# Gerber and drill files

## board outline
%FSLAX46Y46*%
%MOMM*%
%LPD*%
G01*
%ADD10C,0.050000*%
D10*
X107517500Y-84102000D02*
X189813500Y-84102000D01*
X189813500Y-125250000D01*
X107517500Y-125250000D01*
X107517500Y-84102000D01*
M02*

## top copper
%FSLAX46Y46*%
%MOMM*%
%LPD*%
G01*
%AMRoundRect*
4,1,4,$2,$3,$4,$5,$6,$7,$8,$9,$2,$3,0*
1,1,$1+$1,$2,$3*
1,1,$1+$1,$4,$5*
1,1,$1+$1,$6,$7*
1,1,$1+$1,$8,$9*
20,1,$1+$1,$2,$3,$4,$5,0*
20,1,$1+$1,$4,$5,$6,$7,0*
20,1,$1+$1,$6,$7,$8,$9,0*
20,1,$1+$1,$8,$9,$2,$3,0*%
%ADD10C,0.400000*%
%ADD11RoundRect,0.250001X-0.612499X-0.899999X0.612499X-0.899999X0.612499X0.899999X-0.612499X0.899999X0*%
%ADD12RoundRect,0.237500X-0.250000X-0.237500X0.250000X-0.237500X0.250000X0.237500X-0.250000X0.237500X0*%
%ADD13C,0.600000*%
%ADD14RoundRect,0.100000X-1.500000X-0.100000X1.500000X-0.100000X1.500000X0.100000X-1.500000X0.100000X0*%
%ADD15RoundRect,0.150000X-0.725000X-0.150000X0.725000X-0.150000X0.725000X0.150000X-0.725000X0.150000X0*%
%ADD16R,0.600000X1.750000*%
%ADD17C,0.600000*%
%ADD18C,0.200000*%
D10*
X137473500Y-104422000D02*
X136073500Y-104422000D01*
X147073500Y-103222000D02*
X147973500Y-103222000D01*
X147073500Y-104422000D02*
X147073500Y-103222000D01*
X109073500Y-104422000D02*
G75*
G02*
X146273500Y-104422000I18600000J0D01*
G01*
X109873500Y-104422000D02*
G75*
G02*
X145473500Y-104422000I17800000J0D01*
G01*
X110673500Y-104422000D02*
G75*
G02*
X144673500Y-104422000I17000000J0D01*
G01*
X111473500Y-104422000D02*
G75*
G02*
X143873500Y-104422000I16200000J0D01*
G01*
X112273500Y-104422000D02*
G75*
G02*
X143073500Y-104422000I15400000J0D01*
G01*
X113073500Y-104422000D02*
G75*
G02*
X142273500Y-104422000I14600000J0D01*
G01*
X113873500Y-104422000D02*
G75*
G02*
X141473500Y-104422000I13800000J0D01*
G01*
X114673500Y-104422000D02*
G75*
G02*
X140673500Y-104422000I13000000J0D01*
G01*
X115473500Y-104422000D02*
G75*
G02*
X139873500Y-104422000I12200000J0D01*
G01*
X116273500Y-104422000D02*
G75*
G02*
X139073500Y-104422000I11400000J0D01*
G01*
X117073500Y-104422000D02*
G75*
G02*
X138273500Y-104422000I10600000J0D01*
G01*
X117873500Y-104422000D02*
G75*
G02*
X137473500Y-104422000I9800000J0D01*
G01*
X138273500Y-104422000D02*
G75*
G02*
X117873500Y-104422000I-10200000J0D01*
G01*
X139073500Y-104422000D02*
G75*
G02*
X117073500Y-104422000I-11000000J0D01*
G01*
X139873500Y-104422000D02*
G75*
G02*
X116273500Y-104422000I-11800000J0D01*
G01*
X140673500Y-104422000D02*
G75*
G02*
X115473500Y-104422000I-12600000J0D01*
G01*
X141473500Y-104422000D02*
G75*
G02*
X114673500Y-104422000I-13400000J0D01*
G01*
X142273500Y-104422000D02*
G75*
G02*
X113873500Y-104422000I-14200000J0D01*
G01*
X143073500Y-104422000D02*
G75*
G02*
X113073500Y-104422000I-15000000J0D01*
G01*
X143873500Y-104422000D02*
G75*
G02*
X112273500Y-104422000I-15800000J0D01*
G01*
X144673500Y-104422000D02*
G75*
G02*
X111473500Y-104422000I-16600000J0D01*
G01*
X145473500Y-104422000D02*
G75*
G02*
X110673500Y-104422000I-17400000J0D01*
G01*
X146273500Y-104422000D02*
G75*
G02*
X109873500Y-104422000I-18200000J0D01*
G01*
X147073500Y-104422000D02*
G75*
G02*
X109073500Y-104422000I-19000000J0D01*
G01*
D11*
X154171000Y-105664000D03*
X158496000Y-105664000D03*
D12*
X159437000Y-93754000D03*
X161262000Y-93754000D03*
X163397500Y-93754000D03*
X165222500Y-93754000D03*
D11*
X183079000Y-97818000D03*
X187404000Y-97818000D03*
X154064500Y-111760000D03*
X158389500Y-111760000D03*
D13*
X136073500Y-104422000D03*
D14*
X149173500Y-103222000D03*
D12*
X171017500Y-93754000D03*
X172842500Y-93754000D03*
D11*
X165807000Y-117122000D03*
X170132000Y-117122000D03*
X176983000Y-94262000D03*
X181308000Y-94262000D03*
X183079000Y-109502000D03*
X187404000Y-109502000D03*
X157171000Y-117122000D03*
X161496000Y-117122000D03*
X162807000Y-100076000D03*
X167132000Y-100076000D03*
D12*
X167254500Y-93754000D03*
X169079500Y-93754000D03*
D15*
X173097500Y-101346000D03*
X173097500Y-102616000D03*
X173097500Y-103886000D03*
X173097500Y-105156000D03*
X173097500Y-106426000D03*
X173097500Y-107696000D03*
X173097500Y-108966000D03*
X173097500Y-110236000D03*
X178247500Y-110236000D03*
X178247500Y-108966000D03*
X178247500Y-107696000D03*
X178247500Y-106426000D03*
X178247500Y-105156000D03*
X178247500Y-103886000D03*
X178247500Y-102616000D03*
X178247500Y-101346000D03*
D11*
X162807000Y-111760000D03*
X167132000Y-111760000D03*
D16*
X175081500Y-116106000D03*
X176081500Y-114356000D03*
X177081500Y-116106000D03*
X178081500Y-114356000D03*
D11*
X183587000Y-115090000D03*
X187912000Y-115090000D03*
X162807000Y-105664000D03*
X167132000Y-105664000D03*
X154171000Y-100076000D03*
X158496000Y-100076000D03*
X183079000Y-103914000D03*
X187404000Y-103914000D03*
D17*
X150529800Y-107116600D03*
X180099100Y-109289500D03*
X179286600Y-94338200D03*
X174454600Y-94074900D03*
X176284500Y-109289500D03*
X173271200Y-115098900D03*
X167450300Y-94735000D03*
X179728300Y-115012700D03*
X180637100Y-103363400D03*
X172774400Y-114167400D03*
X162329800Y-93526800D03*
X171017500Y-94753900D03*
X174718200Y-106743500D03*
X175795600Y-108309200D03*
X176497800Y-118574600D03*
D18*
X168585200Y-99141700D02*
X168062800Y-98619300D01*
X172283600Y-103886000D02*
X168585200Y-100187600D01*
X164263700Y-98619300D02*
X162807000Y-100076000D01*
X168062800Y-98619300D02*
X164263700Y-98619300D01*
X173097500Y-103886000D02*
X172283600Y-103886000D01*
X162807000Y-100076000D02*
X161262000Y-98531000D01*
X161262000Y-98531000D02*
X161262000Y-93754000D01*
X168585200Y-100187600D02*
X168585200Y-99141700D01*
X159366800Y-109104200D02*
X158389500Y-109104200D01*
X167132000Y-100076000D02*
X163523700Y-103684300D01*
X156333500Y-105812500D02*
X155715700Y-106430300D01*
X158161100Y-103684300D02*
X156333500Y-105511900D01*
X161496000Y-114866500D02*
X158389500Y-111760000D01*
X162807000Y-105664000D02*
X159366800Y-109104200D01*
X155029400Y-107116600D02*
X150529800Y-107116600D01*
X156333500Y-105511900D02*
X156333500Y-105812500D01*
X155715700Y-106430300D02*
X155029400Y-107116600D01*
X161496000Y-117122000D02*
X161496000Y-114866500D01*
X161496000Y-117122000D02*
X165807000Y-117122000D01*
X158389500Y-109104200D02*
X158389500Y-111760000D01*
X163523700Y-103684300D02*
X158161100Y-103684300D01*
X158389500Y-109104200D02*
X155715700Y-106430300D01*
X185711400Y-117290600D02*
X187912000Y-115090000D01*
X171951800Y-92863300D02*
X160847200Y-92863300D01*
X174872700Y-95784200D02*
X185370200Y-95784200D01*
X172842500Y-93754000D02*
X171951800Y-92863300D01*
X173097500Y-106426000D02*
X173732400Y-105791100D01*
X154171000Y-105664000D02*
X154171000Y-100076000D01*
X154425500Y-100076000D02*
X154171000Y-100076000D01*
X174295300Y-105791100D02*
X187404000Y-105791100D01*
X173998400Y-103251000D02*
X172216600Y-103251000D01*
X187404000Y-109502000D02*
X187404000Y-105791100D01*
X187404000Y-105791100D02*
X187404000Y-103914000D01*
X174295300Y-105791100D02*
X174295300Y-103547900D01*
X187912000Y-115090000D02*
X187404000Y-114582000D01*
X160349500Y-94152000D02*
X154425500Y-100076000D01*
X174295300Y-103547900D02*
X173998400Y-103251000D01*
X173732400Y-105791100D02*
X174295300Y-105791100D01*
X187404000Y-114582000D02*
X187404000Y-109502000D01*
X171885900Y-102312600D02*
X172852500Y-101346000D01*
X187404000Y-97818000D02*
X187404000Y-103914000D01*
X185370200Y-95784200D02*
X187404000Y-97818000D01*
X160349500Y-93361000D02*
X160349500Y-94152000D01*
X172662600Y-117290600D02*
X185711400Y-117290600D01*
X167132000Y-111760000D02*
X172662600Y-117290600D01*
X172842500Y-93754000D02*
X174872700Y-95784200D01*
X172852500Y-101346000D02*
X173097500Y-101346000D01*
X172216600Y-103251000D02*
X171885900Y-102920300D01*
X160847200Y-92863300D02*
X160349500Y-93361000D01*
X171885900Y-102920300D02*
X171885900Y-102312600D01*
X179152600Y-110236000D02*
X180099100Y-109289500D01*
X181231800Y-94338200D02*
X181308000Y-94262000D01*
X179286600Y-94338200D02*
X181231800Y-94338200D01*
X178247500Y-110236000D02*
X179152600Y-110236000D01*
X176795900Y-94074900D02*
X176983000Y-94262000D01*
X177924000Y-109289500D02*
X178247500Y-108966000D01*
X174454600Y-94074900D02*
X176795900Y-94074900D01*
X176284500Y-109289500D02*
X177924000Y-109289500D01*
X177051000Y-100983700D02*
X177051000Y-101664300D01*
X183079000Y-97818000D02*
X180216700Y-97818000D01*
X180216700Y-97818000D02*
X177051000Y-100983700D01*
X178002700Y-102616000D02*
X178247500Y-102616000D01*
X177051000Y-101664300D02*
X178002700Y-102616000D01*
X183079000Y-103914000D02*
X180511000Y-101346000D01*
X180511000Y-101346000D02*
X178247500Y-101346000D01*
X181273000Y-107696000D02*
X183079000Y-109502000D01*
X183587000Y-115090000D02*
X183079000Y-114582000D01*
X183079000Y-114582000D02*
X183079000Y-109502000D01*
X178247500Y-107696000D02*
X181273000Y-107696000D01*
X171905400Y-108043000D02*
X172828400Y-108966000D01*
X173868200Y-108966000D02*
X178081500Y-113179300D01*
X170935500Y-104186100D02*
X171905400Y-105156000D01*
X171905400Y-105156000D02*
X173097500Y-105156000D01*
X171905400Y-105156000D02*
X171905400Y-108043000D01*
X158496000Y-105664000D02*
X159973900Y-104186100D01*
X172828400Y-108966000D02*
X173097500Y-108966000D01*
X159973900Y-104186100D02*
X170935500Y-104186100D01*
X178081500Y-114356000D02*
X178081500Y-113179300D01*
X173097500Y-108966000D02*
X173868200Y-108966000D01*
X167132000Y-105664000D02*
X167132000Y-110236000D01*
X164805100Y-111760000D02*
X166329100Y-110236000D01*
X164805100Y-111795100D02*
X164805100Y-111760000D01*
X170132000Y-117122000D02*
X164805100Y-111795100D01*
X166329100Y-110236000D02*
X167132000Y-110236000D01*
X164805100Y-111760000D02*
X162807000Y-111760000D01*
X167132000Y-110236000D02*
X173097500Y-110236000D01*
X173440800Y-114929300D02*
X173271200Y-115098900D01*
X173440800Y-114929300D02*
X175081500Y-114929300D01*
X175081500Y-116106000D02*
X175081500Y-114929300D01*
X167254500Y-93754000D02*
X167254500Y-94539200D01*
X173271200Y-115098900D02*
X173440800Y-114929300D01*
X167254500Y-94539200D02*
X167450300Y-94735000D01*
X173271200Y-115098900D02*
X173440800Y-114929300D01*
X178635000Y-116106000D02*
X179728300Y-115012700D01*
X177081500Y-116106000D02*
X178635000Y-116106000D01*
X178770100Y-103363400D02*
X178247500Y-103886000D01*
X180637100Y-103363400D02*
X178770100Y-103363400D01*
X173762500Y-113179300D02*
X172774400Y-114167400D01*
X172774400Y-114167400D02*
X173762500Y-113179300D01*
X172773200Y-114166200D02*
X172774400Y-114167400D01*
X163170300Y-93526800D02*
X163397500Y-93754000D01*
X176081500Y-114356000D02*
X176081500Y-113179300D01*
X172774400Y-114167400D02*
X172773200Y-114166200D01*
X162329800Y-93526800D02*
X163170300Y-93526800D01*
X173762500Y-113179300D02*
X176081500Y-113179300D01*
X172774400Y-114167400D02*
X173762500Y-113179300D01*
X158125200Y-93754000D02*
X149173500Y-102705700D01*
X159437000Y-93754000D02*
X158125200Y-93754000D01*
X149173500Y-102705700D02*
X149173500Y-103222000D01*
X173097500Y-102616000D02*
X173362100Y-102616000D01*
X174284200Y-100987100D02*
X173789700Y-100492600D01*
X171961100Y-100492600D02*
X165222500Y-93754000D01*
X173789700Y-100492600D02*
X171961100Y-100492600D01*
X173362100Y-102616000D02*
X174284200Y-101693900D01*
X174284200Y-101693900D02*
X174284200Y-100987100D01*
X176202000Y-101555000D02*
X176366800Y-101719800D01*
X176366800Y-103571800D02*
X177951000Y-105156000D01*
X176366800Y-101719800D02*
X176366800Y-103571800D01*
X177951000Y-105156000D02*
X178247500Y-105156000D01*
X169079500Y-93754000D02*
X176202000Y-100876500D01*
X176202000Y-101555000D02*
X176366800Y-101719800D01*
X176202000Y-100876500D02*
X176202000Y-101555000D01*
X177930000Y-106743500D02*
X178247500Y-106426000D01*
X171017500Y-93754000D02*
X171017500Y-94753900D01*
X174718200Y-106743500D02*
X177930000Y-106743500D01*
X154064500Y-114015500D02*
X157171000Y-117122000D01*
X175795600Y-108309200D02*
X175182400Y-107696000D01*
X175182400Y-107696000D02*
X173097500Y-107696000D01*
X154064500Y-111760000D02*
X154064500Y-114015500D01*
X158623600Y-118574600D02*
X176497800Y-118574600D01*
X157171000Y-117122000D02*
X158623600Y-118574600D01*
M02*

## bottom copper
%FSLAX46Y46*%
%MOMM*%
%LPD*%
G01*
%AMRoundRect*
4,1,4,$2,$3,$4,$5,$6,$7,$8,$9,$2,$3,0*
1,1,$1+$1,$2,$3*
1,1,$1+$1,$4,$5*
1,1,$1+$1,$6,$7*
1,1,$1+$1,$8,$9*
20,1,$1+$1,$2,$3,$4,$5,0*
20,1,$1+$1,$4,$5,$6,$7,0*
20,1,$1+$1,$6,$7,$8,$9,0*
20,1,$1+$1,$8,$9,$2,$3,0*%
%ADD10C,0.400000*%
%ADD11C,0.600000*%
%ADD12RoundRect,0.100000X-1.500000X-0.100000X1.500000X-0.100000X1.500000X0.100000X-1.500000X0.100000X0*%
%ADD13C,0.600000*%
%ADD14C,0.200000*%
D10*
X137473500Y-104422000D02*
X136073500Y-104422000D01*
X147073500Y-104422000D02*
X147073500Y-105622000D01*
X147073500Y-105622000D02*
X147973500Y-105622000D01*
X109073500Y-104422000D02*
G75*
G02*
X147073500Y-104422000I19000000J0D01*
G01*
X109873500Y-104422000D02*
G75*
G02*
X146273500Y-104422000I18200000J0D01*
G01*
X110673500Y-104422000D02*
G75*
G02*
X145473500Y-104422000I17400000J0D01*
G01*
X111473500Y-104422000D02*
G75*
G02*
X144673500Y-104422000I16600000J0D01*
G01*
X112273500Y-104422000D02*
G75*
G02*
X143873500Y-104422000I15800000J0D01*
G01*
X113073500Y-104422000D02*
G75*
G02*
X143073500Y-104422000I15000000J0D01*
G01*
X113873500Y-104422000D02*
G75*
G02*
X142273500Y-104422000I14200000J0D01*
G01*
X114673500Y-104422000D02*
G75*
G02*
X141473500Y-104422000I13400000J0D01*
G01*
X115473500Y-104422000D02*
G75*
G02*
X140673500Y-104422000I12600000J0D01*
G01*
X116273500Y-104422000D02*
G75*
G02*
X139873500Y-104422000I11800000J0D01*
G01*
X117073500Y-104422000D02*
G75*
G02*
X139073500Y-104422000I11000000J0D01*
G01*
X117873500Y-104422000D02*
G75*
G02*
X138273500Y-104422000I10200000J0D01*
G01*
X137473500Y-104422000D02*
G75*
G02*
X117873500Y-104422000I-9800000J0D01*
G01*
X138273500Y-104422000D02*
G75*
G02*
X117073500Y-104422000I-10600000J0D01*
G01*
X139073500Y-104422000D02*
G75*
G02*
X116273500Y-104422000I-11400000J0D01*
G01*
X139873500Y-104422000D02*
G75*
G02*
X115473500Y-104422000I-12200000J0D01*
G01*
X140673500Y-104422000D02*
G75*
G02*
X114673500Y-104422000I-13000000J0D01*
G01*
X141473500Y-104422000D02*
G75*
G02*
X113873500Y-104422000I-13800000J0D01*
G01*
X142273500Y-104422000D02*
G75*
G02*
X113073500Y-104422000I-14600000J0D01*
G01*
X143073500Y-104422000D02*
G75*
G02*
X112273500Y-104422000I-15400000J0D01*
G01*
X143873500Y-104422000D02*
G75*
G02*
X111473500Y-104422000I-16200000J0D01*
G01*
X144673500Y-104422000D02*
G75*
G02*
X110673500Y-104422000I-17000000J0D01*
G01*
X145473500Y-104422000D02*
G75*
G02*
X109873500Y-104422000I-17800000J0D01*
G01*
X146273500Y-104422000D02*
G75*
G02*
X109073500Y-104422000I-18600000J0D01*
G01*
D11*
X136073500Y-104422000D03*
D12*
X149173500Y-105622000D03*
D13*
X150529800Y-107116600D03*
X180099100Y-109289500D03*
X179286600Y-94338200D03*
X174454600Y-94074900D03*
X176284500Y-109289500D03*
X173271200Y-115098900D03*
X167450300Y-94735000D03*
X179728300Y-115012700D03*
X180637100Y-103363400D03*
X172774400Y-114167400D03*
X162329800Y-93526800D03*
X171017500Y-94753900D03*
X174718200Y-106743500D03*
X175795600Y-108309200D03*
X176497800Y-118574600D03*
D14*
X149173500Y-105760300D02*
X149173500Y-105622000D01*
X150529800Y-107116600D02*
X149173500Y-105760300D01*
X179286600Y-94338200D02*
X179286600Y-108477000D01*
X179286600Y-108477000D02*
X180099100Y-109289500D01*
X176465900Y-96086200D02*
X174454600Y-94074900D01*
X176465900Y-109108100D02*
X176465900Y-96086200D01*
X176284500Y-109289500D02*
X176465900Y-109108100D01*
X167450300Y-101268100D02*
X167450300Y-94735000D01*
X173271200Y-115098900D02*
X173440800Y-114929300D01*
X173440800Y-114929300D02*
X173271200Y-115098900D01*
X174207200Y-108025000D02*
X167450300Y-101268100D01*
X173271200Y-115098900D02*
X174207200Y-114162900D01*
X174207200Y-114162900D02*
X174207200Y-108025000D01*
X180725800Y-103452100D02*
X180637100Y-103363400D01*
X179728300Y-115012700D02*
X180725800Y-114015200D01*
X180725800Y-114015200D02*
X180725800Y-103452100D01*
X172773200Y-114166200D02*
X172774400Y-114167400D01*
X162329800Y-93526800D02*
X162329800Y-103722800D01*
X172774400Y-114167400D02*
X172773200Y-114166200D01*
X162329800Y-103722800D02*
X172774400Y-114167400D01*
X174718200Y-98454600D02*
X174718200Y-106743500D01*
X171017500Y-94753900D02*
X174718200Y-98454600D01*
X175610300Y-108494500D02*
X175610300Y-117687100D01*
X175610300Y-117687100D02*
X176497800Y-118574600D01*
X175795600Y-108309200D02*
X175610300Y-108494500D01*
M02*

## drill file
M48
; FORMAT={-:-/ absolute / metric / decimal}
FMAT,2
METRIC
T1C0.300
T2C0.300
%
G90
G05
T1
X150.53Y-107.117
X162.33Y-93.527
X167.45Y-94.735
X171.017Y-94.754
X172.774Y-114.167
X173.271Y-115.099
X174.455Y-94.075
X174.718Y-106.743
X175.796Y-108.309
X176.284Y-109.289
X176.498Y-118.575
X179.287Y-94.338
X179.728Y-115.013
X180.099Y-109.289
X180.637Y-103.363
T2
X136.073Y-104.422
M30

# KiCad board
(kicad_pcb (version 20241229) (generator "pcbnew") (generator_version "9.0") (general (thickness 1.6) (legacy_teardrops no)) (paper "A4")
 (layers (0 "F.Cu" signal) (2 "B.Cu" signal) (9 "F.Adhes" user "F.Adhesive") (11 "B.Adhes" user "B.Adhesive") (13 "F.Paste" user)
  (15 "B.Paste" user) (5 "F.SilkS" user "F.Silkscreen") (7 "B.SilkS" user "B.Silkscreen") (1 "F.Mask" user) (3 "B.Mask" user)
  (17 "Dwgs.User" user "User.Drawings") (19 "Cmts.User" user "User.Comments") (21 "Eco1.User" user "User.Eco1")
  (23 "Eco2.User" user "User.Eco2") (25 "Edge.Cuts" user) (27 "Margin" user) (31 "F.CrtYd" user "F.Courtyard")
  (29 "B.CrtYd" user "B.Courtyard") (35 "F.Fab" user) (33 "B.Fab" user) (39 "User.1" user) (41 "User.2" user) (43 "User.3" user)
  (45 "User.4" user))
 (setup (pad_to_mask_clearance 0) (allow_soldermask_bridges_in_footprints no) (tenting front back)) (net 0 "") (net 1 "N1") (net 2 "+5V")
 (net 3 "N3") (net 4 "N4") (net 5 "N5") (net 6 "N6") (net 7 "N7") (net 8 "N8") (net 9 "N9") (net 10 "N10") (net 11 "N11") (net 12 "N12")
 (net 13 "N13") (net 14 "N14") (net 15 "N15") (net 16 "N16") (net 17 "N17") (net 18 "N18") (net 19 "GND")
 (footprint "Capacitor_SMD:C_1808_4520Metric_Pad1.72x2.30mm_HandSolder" (layer "F.Cu") (at 156.3335 105.664)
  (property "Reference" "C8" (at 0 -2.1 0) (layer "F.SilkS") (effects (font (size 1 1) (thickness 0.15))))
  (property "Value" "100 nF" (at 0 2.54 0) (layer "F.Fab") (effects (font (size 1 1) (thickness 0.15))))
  (pad "1" smd roundrect (at -2.1625 0) (size 1.725 2.3) (layers "F.Cu" "F.Mask" "F.Paste") (roundrect_rratio 0.144928) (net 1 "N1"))
  (pad "2" smd roundrect (at 2.1625 0) (size 1.725 2.3) (layers "F.Cu" "F.Mask" "F.Paste") (roundrect_rratio 0.144928) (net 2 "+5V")))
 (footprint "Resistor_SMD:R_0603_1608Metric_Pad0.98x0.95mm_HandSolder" (layer "F.Cu") (at 160.3495 93.754)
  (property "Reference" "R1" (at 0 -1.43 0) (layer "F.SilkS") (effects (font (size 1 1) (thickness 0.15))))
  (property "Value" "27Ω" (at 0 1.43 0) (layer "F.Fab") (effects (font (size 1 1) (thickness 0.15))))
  (pad "1" smd roundrect (at -0.9125 0) (size 0.975 0.95) (layers "F.Cu" "F.Mask" "F.Paste") (roundrect_rratio 0.25) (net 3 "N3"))
  (pad "2" smd roundrect (at 0.9125 0) (size 0.975 0.95) (layers "F.Cu" "F.Mask" "F.Paste") (roundrect_rratio 0.25) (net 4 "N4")))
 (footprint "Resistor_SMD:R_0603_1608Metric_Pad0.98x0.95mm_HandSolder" (layer "F.Cu") (at 164.31 93.754)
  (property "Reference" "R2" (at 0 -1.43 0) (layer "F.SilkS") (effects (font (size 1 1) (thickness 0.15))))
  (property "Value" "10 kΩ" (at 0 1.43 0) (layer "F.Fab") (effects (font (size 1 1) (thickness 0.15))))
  (pad "1" smd roundrect (at -0.9125 0) (size 0.975 0.95) (layers "F.Cu" "F.Mask" "F.Paste") (roundrect_rratio 0.25) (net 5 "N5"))
  (pad "2" smd roundrect (at 0.9125 0) (size 0.975 0.95) (layers "F.Cu" "F.Mask" "F.Paste") (roundrect_rratio 0.25) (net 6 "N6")))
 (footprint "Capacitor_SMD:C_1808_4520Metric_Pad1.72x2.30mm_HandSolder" (layer "F.Cu") (at 185.2415 97.818)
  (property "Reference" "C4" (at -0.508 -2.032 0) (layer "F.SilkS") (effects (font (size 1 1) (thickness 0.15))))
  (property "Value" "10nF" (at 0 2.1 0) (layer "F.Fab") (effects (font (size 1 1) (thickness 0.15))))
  (pad "1" smd roundrect (at -2.1625 0) (size 1.725 2.3) (layers "F.Cu" "F.Mask" "F.Paste") (roundrect_rratio 0.144928) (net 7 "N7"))
  (pad "2" smd roundrect (at 2.1625 0) (size 1.725 2.3) (layers "F.Cu" "F.Mask" "F.Paste") (roundrect_rratio 0.144928) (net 1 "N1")))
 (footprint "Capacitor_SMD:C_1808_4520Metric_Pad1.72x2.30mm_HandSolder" (layer "F.Cu") (at 156.227 111.76)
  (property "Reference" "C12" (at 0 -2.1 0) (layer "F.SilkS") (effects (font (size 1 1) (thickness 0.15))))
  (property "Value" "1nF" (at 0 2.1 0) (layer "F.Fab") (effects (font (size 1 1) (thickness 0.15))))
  (pad "1" smd roundrect (at -2.1625 0) (size 1.725 2.3) (layers "F.Cu" "F.Mask" "F.Paste") (roundrect_rratio 0.144928) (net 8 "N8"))
  (pad "2" smd roundrect (at 2.1625 0) (size 1.725 2.3) (layers "F.Cu" "F.Mask" "F.Paste") (roundrect_rratio 0.144928) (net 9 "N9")))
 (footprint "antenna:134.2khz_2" (layer "F.Cu") (at 127.6735 104.422)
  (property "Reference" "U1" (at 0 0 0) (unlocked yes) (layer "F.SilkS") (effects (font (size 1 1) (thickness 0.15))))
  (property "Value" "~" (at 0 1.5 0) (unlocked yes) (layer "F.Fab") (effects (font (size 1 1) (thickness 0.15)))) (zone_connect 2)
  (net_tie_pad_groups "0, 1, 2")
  (fp_line (start 9.8 0) (end 8.4 0) (stroke (width 0.4) (type default)) (layer "F.Cu"))
  (fp_line (start 19.4 -1.2) (end 20.3 -1.2) (stroke (width 0.4) (type default)) (layer "F.Cu"))
  (fp_line (start 19.4 0) (end 19.4 -1.2) (stroke (width 0.4) (type default)) (layer "F.Cu"))
  (fp_arc (start -18.6 0) (mid 0 -18.6) (end 18.6 0) (stroke (width 0.4) (type default)) (layer "F.Cu"))
  (fp_arc (start -17.8 0) (mid 0 -17.8) (end 17.8 0) (stroke (width 0.4) (type default)) (layer "F.Cu"))
  (fp_arc (start -17 0) (mid 0 -17) (end 17 0) (stroke (width 0.4) (type default)) (layer "F.Cu"))
  (fp_arc (start -16.2 0) (mid 0 -16.2) (end 16.2 0) (stroke (width 0.4) (type default)) (layer "F.Cu"))
  (fp_arc (start -15.4 0) (mid 0 -15.4) (end 15.4 0) (stroke (width 0.4) (type default)) (layer "F.Cu"))
  (fp_arc (start -14.6 0) (mid 0 -14.6) (end 14.6 0) (stroke (width 0.4) (type default)) (layer "F.Cu"))
  (fp_arc (start -13.8 0) (mid 0 -13.8) (end 13.8 0) (stroke (width 0.4) (type default)) (layer "F.Cu"))
  (fp_arc (start -13 0) (mid 0 -13) (end 13 0) (stroke (width 0.4) (type default)) (layer "F.Cu"))
  (fp_arc (start -12.2 0) (mid 0 -12.2) (end 12.2 0) (stroke (width 0.4) (type default)) (layer "F.Cu"))
  (fp_arc (start -11.4 0) (mid 0 -11.4) (end 11.4 0) (stroke (width 0.4) (type default)) (layer "F.Cu"))
  (fp_arc (start -10.6 0) (mid 0 -10.6) (end 10.6 0) (stroke (width 0.4) (type default)) (layer "F.Cu"))
  (fp_arc (start -9.8 0) (mid 0 -9.8) (end 9.8 0) (stroke (width 0.4) (type default)) (layer "F.Cu"))
  (fp_arc (start 10.6 0) (mid 0.4 10.2) (end -9.8 0) (stroke (width 0.4) (type default)) (layer "F.Cu"))
  (fp_arc (start 11.4 0) (mid 0.4 11) (end -10.6 0) (stroke (width 0.4) (type default)) (layer "F.Cu"))
  (fp_arc (start 12.2 0) (mid 0.4 11.8) (end -11.4 0) (stroke (width 0.4) (type default)) (layer "F.Cu"))
  (fp_arc (start 13 0) (mid 0.4 12.6) (end -12.2 0) (stroke (width 0.4) (type default)) (layer "F.Cu"))
  (fp_arc (start 13.8 0) (mid 0.4 13.4) (end -13 0) (stroke (width 0.4) (type default)) (layer "F.Cu"))
  (fp_arc (start 14.6 0) (mid 0.4 14.2) (end -13.8 0) (stroke (width 0.4) (type default)) (layer "F.Cu"))
  (fp_arc (start 15.4 0) (mid 0.4 15) (end -14.6 0) (stroke (width 0.4) (type default)) (layer "F.Cu"))
  (fp_arc (start 16.2 0) (mid 0.4 15.8) (end -15.4 0) (stroke (width 0.4) (type default)) (layer "F.Cu"))
  (fp_arc (start 17 0) (mid 0.4 16.6) (end -16.2 0) (stroke (width 0.4) (type default)) (layer "F.Cu"))
  (fp_arc (start 17.8 0) (mid 0.4 17.4) (end -17 0) (stroke (width 0.4) (type default)) (layer "F.Cu"))
  (fp_arc (start 18.6 0) (mid 0.4 18.2) (end -17.8 0) (stroke (width 0.4) (type default)) (layer "F.Cu"))
  (fp_arc (start 19.4 0) (mid 0.4 19) (end -18.6 0) (stroke (width 0.4) (type default)) (layer "F.Cu"))
  (fp_line (start 9.8 0) (end 8.4 0) (stroke (width 0.4) (type default)) (layer "B.Cu"))
  (fp_line (start 19.4 0) (end 19.4 1.2) (stroke (width 0.4) (type default)) (layer "B.Cu"))
  (fp_line (start 19.4 1.2) (end 20.3 1.2) (stroke (width 0.4) (type default)) (layer "B.Cu"))
  (fp_arc (start -18.6 0) (mid 0.4 -19) (end 19.4 0) (stroke (width 0.4) (type default)) (layer "B.Cu"))
  (fp_arc (start -17.8 0) (mid 0.4 -18.2) (end 18.6 0) (stroke (width 0.4) (type default)) (layer "B.Cu"))
  (fp_arc (start -17 0) (mid 0.4 -17.4) (end 17.8 0) (stroke (width 0.4) (type default)) (layer "B.Cu"))
  (fp_arc (start -16.2 0) (mid 0.4 -16.6) (end 17 0) (stroke (width 0.4) (type default)) (layer "B.Cu"))
  (fp_arc (start -15.4 0) (mid 0.4 -15.8) (end 16.2 0) (stroke (width 0.4) (type default)) (layer "B.Cu"))
  (fp_arc (start -14.6 0) (mid 0.4 -15) (end 15.4 0) (stroke (width 0.4) (type default)) (layer "B.Cu"))
  (fp_arc (start -13.8 0) (mid 0.4 -14.2) (end 14.6 0) (stroke (width 0.4) (type default)) (layer "B.Cu"))
  (fp_arc (start -13 0) (mid 0.4 -13.4) (end 13.8 0) (stroke (width 0.4) (type default)) (layer "B.Cu"))
  (fp_arc (start -12.2 0) (mid 0.4 -12.6) (end 13 0) (stroke (width 0.4) (type default)) (layer "B.Cu"))
  (fp_arc (start -11.4 0) (mid 0.4 -11.8) (end 12.2 0) (stroke (width 0.4) (type default)) (layer "B.Cu"))
  (fp_arc (start -10.6 0) (mid 0.4 -11) (end 11.4 0) (stroke (width 0.4) (type default)) (layer "B.Cu"))
  (fp_arc (start -9.8 0) (mid 0.4 -10.2) (end 10.6 0) (stroke (width 0.4) (type default)) (layer "B.Cu"))
  (fp_arc (start 9.8 0) (mid 0 9.8) (end -9.8 0) (stroke (width 0.4) (type default)) (layer "B.Cu"))
  (fp_arc (start 10.6 0) (mid 0 10.6) (end -10.6 0) (stroke (width 0.4) (type default)) (layer "B.Cu"))
  (fp_arc (start 11.4 0) (mid 0 11.4) (end -11.4 0) (stroke (width 0.4) (type default)) (layer "B.Cu"))
  (fp_arc (start 12.2 0) (mid 0 12.2) (end -12.2 0) (stroke (width 0.4) (type default)) (layer "B.Cu"))
  (fp_arc (start 13 0) (mid 0 13) (end -13 0) (stroke (width 0.4) (type default)) (layer "B.Cu"))
  (fp_arc (start 13.8 0) (mid 0 13.8) (end -13.8 0) (stroke (width 0.4) (type default)) (layer "B.Cu"))
  (fp_arc (start 14.6 0) (mid 0 14.6) (end -14.6 0) (stroke (width 0.4) (type default)) (layer "B.Cu"))
  (fp_arc (start 15.4 0) (mid 0 15.4) (end -15.4 0) (stroke (width 0.4) (type default)) (layer "B.Cu"))
  (fp_arc (start 16.2 0) (mid 0 16.2) (end -16.2 0) (stroke (width 0.4) (type default)) (layer "B.Cu"))
  (fp_arc (start 17 0) (mid 0 17) (end -17 0) (stroke (width 0.4) (type default)) (layer "B.Cu"))
  (fp_arc (start 17.8 0) (mid 0 17.8) (end -17.8 0) (stroke (width 0.4) (type default)) (layer "B.Cu"))
  (fp_arc (start 18.6 0) (mid 0 18.6) (end -18.6 0) (stroke (width 0.4) (type default)) (layer "B.Cu"))
  (pad "0" thru_hole circle (at 8.4 0) (size 0.6 0.6) (drill 0.3) (layers "*.Cu") (remove_unused_layers yes) (keep_end_layers yes)
   (zone_layer_connections))
  (pad "1" smd roundrect (at 21.5 -1.2) (size 3.2 0.4) (layers "F.Cu") (roundrect_rratio 0.25) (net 3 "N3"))
  (pad "2" smd roundrect (at 21.5 1.2) (size 3.2 0.4) (layers "B.Cu") (roundrect_rratio 0.25) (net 9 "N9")))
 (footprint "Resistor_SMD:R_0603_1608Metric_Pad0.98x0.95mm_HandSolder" (layer "F.Cu") (at 171.93 93.754)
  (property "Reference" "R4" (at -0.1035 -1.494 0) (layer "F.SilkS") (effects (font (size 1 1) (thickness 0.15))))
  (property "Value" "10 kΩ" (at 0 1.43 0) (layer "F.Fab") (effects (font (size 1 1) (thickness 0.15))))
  (pad "1" smd roundrect (at -0.9125 0) (size 0.975 0.95) (layers "F.Cu" "F.Mask" "F.Paste") (roundrect_rratio 0.25) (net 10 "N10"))
  (pad "2" smd roundrect (at 0.9125 0) (size 0.975 0.95) (layers "F.Cu" "F.Mask" "F.Paste") (roundrect_rratio 0.25) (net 1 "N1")))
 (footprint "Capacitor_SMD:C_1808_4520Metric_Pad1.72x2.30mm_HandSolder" (layer "F.Cu") (at 167.9695 117.122)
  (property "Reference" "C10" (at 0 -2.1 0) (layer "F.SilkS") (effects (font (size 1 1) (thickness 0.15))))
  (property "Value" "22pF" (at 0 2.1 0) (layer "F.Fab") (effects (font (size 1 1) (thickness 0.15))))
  (pad "1" smd roundrect (at -2.1625 0) (size 1.725 2.3) (layers "F.Cu" "F.Mask" "F.Paste") (roundrect_rratio 0.144928) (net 9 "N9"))
  (pad "2" smd roundrect (at 2.1625 0) (size 1.725 2.3) (layers "F.Cu" "F.Mask" "F.Paste") (roundrect_rratio 0.144928) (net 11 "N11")))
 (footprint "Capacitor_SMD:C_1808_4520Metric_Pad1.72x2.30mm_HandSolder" (layer "F.Cu") (at 179.1455 94.262)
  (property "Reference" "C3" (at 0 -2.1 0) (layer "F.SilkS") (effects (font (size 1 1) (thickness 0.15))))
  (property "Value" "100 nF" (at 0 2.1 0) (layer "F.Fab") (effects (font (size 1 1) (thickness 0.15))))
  (pad "1" smd roundrect (at -2.1625 0) (size 1.725 2.3) (layers "F.Cu" "F.Mask" "F.Paste") (roundrect_rratio 0.144928) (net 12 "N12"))
  (pad "2" smd roundrect (at 2.1625 0) (size 1.725 2.3) (layers "F.Cu" "F.Mask" "F.Paste") (roundrect_rratio 0.144928) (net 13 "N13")))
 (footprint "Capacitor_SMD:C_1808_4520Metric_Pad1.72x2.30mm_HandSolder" (layer "F.Cu") (at 185.2415 109.502)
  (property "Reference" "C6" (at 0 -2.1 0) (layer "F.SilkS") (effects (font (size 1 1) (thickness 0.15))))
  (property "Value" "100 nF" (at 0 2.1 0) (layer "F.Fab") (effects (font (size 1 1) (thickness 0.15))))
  (pad "1" smd roundrect (at -2.1625 0) (size 1.725 2.3) (layers "F.Cu" "F.Mask" "F.Paste") (roundrect_rratio 0.144928) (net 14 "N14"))
  (pad "2" smd roundrect (at 2.1625 0) (size 1.725 2.3) (layers "F.Cu" "F.Mask" "F.Paste") (roundrect_rratio 0.144928) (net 1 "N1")))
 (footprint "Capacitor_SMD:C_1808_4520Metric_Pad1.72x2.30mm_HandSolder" (layer "F.Cu") (at 159.3335 117.122)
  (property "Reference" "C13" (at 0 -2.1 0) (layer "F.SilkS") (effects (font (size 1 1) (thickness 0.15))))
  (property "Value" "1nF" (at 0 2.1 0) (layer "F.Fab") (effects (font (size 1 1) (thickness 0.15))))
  (pad "1" smd roundrect (at -2.1625 0) (size 1.725 2.3) (layers "F.Cu" "F.Mask" "F.Paste") (roundrect_rratio 0.144928) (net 8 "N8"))
  (pad "2" smd roundrect (at 2.1625 0) (size 1.725 2.3) (layers "F.Cu" "F.Mask" "F.Paste") (roundrect_rratio 0.144928) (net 9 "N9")))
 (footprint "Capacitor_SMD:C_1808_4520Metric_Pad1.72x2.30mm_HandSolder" (layer "F.Cu") (at 164.9695 100.076)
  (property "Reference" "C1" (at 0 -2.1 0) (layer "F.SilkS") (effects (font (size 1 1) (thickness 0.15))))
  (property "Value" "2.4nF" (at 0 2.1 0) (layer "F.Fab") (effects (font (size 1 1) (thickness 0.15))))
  (pad "1" smd roundrect (at -2.1625 0) (size 1.725 2.3) (layers "F.Cu" "F.Mask" "F.Paste") (roundrect_rratio 0.144928) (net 4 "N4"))
  (pad "2" smd roundrect (at 2.1625 0) (size 1.725 2.3) (layers "F.Cu" "F.Mask" "F.Paste") (roundrect_rratio 0.144928) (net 9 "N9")))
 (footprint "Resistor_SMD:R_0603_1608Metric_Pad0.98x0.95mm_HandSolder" (layer "F.Cu") (at 168.167 93.754)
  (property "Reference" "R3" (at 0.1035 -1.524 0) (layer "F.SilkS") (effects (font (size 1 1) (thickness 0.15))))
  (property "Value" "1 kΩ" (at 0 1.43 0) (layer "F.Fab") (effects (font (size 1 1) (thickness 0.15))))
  (pad "1" smd roundrect (at -0.9125 0) (size 0.975 0.95) (layers "F.Cu" "F.Mask" "F.Paste") (roundrect_rratio 0.25) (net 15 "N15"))
  (pad "2" smd roundrect (at 0.9125 0) (size 0.975 0.95) (layers "F.Cu" "F.Mask" "F.Paste") (roundrect_rratio 0.25) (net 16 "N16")))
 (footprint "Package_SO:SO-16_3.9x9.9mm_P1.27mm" (layer "F.Cu") (at 175.6725 105.791)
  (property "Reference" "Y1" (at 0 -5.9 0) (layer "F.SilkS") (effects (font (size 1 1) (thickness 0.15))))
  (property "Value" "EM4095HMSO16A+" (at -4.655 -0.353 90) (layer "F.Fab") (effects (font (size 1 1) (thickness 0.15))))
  (pad "1" smd roundrect (at -2.575 -4.445) (size 1.75 0.6) (layers "F.Cu" "F.Mask" "F.Paste") (roundrect_rratio 0.25) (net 1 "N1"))
  (pad "2" smd roundrect (at -2.575 -3.175) (size 1.75 0.6) (layers "F.Cu" "F.Mask" "F.Paste") (roundrect_rratio 0.25) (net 6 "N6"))
  (pad "3" smd roundrect (at -2.575 -1.905) (size 1.75 0.6) (layers "F.Cu" "F.Mask" "F.Paste") (roundrect_rratio 0.25) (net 4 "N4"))
  (pad "4" smd roundrect (at -2.575 -0.635) (size 1.75 0.6) (layers "F.Cu" "F.Mask" "F.Paste") (roundrect_rratio 0.25) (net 2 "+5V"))
  (pad "5" smd roundrect (at -2.575 0.635) (size 1.75 0.6) (layers "F.Cu" "F.Mask" "F.Paste") (roundrect_rratio 0.25) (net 1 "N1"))
  (pad "6" smd roundrect (at -2.575 1.905) (size 1.75 0.6) (layers "F.Cu" "F.Mask" "F.Paste") (roundrect_rratio 0.25) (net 8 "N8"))
  (pad "7" smd roundrect (at -2.575 3.175) (size 1.75 0.6) (layers "F.Cu" "F.Mask" "F.Paste") (roundrect_rratio 0.25) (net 2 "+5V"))
  (pad "8" smd roundrect (at -2.575 4.445) (size 1.75 0.6) (layers "F.Cu" "F.Mask" "F.Paste") (roundrect_rratio 0.25) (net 11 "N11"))
  (pad "9" smd roundrect (at 2.575 4.445) (size 1.75 0.6) (layers "F.Cu" "F.Mask" "F.Paste") (roundrect_rratio 0.25) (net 13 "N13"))
  (pad "10" smd roundrect (at 2.575 3.175) (size 1.75 0.6) (layers "F.Cu" "F.Mask" "F.Paste") (roundrect_rratio 0.25) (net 12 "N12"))
  (pad "11" smd roundrect (at 2.575 1.905) (size 1.75 0.6) (layers "F.Cu" "F.Mask" "F.Paste") (roundrect_rratio 0.25) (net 14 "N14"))
  (pad "12" smd roundrect (at 2.575 0.635) (size 1.75 0.6) (layers "F.Cu" "F.Mask" "F.Paste") (roundrect_rratio 0.25) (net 10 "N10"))
  (pad "13" smd roundrect (at 2.575 -0.635) (size 1.75 0.6) (layers "F.Cu" "F.Mask" "F.Paste") (roundrect_rratio 0.25) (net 16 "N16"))
  (pad "14" smd roundrect (at 2.575 -1.905) (size 1.75 0.6) (layers "F.Cu" "F.Mask" "F.Paste") (roundrect_rratio 0.25) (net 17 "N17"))
  (pad "15" smd roundrect (at 2.575 -3.175) (size 1.75 0.6) (layers "F.Cu" "F.Mask" "F.Paste") (roundrect_rratio 0.25) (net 7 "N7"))
  (pad "16" smd roundrect (at 2.575 -4.445) (size 1.75 0.6) (layers "F.Cu" "F.Mask" "F.Paste") (roundrect_rratio 0.25) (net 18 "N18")))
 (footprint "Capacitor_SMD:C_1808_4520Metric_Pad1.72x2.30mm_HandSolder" (layer "F.Cu") (at 164.9695 111.76)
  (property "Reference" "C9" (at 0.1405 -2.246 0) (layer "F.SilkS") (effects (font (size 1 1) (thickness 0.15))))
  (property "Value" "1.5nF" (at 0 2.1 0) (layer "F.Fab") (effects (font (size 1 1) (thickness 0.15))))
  (pad "1" smd roundrect (at -2.1625 0) (size 1.725 2.3) (layers "F.Cu" "F.Mask" "F.Paste") (roundrect_rratio 0.144928) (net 11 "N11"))
  (pad "2" smd roundrect (at 2.1625 0) (size 1.725 2.3) (layers "F.Cu" "F.Mask" "F.Paste") (roundrect_rratio 0.144928) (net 1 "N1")))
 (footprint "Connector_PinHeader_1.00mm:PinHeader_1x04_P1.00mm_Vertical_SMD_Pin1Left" (layer "F.Cu") (at 176.5815 115.231 90)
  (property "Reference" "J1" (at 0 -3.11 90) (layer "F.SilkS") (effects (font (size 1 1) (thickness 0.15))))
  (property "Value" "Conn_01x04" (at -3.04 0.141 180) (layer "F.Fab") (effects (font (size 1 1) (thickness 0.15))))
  (pad "1" smd rect (at -0.875 -1.5 90) (size 1.75 0.6) (layers "F.Cu" "F.Mask" "F.Paste") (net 15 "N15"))
  (pad "2" smd rect (at 0.875 -0.5 90) (size 1.75 0.6) (layers "F.Cu" "F.Mask" "F.Paste") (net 5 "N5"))
  (pad "3" smd rect (at -0.875 0.5 90) (size 1.75 0.6) (layers "F.Cu" "F.Mask" "F.Paste") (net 17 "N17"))
  (pad "4" smd rect (at 0.875 1.5 90) (size 1.75 0.6) (layers "F.Cu" "F.Mask" "F.Paste") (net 2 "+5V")))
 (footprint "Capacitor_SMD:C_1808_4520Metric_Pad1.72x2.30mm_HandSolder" (layer "F.Cu") (at 185.7495 115.09)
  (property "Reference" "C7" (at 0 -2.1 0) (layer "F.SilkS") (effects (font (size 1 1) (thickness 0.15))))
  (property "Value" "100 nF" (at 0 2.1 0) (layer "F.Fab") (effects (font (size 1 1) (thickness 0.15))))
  (pad "1" smd roundrect (at -2.1625 0) (size 1.725 2.3) (layers "F.Cu" "F.Mask" "F.Paste") (roundrect_rratio 0.144928) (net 14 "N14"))
  (pad "2" smd roundrect (at 2.1625 0) (size 1.725 2.3) (layers "F.Cu" "F.Mask" "F.Paste") (roundrect_rratio 0.144928) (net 1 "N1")))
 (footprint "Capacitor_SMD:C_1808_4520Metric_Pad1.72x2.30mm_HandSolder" (layer "F.Cu") (at 164.9695 105.664)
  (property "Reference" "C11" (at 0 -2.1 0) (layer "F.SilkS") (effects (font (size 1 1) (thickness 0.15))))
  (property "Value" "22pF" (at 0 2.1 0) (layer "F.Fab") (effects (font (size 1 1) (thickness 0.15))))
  (pad "1" smd roundrect (at -2.1625 0) (size 1.725 2.3) (layers "F.Cu" "F.Mask" "F.Paste") (roundrect_rratio 0.144928) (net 9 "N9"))
  (pad "2" smd roundrect (at 2.1625 0) (size 1.725 2.3) (layers "F.Cu" "F.Mask" "F.Paste") (roundrect_rratio 0.144928) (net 11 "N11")))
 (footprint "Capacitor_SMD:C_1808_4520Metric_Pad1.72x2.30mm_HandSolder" (layer "F.Cu") (at 156.3335 100.076)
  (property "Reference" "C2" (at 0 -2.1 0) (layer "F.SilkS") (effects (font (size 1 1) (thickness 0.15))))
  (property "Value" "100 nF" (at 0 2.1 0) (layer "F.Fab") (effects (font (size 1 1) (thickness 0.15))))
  (pad "1" smd roundrect (at -2.1625 0) (size 1.725 2.3) (layers "F.Cu" "F.Mask" "F.Paste") (roundrect_rratio 0.144928) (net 1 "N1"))
  (pad "2" smd roundrect (at 2.1625 0) (size 1.725 2.3) (layers "F.Cu" "F.Mask" "F.Paste") (roundrect_rratio 0.144928) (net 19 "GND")))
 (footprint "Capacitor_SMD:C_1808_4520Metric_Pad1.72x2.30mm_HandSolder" (layer "F.Cu") (at 185.2415 103.914)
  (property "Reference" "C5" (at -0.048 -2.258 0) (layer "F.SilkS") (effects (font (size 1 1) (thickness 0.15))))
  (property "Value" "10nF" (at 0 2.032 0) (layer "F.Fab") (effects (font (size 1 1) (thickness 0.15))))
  (pad "1" smd roundrect (at -2.1625 0) (size 1.725 2.3) (layers "F.Cu" "F.Mask" "F.Paste") (roundrect_rratio 0.144928) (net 18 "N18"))
  (pad "2" smd roundrect (at 2.1625 0) (size 1.725 2.3) (layers "F.Cu" "F.Mask" "F.Paste") (roundrect_rratio 0.144928) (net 1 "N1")))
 (gr_rect (start 107.5175 84.102) (end 189.8135 125.25) (stroke (width 0.05) (type default)) (fill no) (layer "Edge.Cuts"))
 (segment (start 168.5852 99.1417) (end 168.0628 98.6193) (width 0.2) (layer "F.Cu") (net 4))
 (segment (start 172.2836 103.886) (end 168.5852 100.1876) (width 0.2) (layer "F.Cu") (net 4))
 (segment (start 164.2637 98.6193) (end 162.807 100.076) (width 0.2) (layer "F.Cu") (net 4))
 (segment (start 168.0628 98.6193) (end 164.2637 98.6193) (width 0.2) (layer "F.Cu") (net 4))
 (segment (start 173.0975 103.886) (end 172.2836 103.886) (width 0.2) (layer "F.Cu") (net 4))
 (segment (start 162.807 100.076) (end 161.262 98.531) (width 0.2) (layer "F.Cu") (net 4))
 (segment (start 161.262 98.531) (end 161.262 93.754) (width 0.2) (layer "F.Cu") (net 4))
 (segment (start 168.5852 100.1876) (end 168.5852 99.1417) (width 0.2) (layer "F.Cu") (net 4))
 (segment (start 159.3668 109.1042) (end 158.3895 109.1042) (width 0.2) (layer "F.Cu") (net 9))
 (segment (start 167.132 100.076) (end 163.5237 103.6843) (width 0.2) (layer "F.Cu") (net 9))
 (segment (start 156.3335 105.8125) (end 155.7157 106.4303) (width 0.2) (layer "F.Cu") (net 9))
 (segment (start 158.1611 103.6843) (end 156.3335 105.5119) (width 0.2) (layer "F.Cu") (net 9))
 (segment (start 161.496 114.8665) (end 158.3895 111.76) (width 0.2) (layer "F.Cu") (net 9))
 (segment (start 162.807 105.664) (end 159.3668 109.1042) (width 0.2) (layer "F.Cu") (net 9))
 (segment (start 155.0294 107.1166) (end 150.5298 107.1166) (width 0.2) (layer "F.Cu") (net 9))
 (segment (start 156.3335 105.5119) (end 156.3335 105.8125) (width 0.2) (layer "F.Cu") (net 9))
 (segment (start 155.7157 106.4303) (end 155.0294 107.1166) (width 0.2) (layer "F.Cu") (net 9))
 (segment (start 161.496 117.122) (end 161.496 114.8665) (width 0.2) (layer "F.Cu") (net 9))
 (segment (start 161.496 117.122) (end 165.807 117.122) (width 0.2) (layer "F.Cu") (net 9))
 (segment (start 158.3895 109.1042) (end 158.3895 111.76) (width 0.2) (layer "F.Cu") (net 9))
 (segment (start 163.5237 103.6843) (end 158.1611 103.6843) (width 0.2) (layer "F.Cu") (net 9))
 (segment (start 158.3895 109.1042) (end 155.7157 106.4303) (width 0.2) (layer "F.Cu") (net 9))
 (via (at 150.5298 107.1166) (size 0.6) (drill 0.3) (layers "F.Cu" "B.Cu") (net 9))
 (segment (start 149.1735 105.7603) (end 149.1735 105.622) (width 0.2) (layer "B.Cu") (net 9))
 (segment (start 150.5298 107.1166) (end 149.1735 105.7603) (width 0.2) (layer "B.Cu") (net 9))
 (segment (start 185.7114 117.2906) (end 187.912 115.09) (width 0.2) (layer "F.Cu") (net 1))
 (segment (start 171.9518 92.8633) (end 160.8472 92.8633) (width 0.2) (layer "F.Cu") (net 1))
 (segment (start 174.8727 95.7842) (end 185.3702 95.7842) (width 0.2) (layer "F.Cu") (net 1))
 (segment (start 172.8425 93.754) (end 171.9518 92.8633) (width 0.2) (layer "F.Cu") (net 1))
 (segment (start 173.0975 106.426) (end 173.7324 105.7911) (width 0.2) (layer "F.Cu") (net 1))
 (segment (start 154.171 105.664) (end 154.171 100.076) (width 0.2) (layer "F.Cu") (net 1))
 (segment (start 154.4255 100.076) (end 154.171 100.076) (width 0.2) (layer "F.Cu") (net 1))
 (segment (start 174.2953 105.7911) (end 187.404 105.7911) (width 0.2) (layer "F.Cu") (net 1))
 (segment (start 173.9984 103.251) (end 172.2166 103.251) (width 0.2) (layer "F.Cu") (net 1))
 (segment (start 187.404 109.502) (end 187.404 105.7911) (width 0.2) (layer "F.Cu") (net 1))
 (segment (start 187.404 105.7911) (end 187.404 103.914) (width 0.2) (layer "F.Cu") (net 1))
 (segment (start 174.2953 105.7911) (end 174.2953 103.5479) (width 0.2) (layer "F.Cu") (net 1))
 (segment (start 187.912 115.09) (end 187.404 114.582) (width 0.2) (layer "F.Cu") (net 1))
 (segment (start 160.3495 94.152) (end 154.4255 100.076) (width 0.2) (layer "F.Cu") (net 1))
 (segment (start 174.2953 103.5479) (end 173.9984 103.251) (width 0.2) (layer "F.Cu") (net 1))
 (segment (start 173.7324 105.7911) (end 174.2953 105.7911) (width 0.2) (layer "F.Cu") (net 1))
 (segment (start 187.404 114.582) (end 187.404 109.502) (width 0.2) (layer "F.Cu") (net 1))
 (segment (start 171.8859 102.3126) (end 172.8525 101.346) (width 0.2) (layer "F.Cu") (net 1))
 (segment (start 187.404 97.818) (end 187.404 103.914) (width 0.2) (layer "F.Cu") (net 1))
 (segment (start 185.3702 95.7842) (end 187.404 97.818) (width 0.2) (layer "F.Cu") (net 1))
 (segment (start 160.3495 93.361) (end 160.3495 94.152) (width 0.2) (layer "F.Cu") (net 1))
 (segment (start 172.6626 117.2906) (end 185.7114 117.2906) (width 0.2) (layer "F.Cu") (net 1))
 (segment (start 167.132 111.76) (end 172.6626 117.2906) (width 0.2) (layer "F.Cu") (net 1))
 (segment (start 172.8425 93.754) (end 174.8727 95.7842) (width 0.2) (layer "F.Cu") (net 1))
 (segment (start 172.8525 101.346) (end 173.0975 101.346) (width 0.2) (layer "F.Cu") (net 1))
 (segment (start 172.2166 103.251) (end 171.8859 102.9203) (width 0.2) (layer "F.Cu") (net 1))
 (segment (start 160.8472 92.8633) (end 160.3495 93.361) (width 0.2) (layer "F.Cu") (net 1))
 (segment (start 171.8859 102.9203) (end 171.8859 102.3126) (width 0.2) (layer "F.Cu") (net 1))
 (segment (start 179.1526 110.236) (end 180.0991 109.2895) (width 0.2) (layer "F.Cu") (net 13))
 (segment (start 181.2318 94.3382) (end 181.308 94.262) (width 0.2) (layer "F.Cu") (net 13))
 (segment (start 179.2866 94.3382) (end 181.2318 94.3382) (width 0.2) (layer "F.Cu") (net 13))
 (segment (start 178.2475 110.236) (end 179.1526 110.236) (width 0.2) (layer "F.Cu") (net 13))
 (via (at 180.0991 109.2895) (size 0.6) (drill 0.3) (layers "F.Cu" "B.Cu") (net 13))
 (via (at 179.2866 94.3382) (size 0.6) (drill 0.3) (layers "F.Cu" "B.Cu") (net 13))
 (segment (start 179.2866 94.3382) (end 179.2866 108.477) (width 0.2) (layer "B.Cu") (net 13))
 (segment (start 179.2866 108.477) (end 180.0991 109.2895) (width 0.2) (layer "B.Cu") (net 13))
 (segment (start 176.7959 94.0749) (end 176.983 94.262) (width 0.2) (layer "F.Cu") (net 12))
 (segment (start 177.924 109.2895) (end 178.2475 108.966) (width 0.2) (layer "F.Cu") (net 12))
 (segment (start 174.4546 94.0749) (end 176.7959 94.0749) (width 0.2) (layer "F.Cu") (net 12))
 (segment (start 176.2845 109.2895) (end 177.924 109.2895) (width 0.2) (layer "F.Cu") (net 12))
 (via (at 174.4546 94.0749) (size 0.6) (drill 0.3) (layers "F.Cu" "B.Cu") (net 12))
 (via (at 176.2845 109.2895) (size 0.6) (drill 0.3) (layers "F.Cu" "B.Cu") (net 12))
 (segment (start 176.4659 96.0862) (end 174.4546 94.0749) (width 0.2) (layer "B.Cu") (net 12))
 (segment (start 176.4659 109.1081) (end 176.4659 96.0862) (width 0.2) (layer "B.Cu") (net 12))
 (segment (start 176.2845 109.2895) (end 176.4659 109.1081) (width 0.2) (layer "B.Cu") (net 12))
 (segment (start 177.051 100.9837) (end 177.051 101.6643) (width 0.2) (layer "F.Cu") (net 7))
 (segment (start 183.079 97.818) (end 180.2167 97.818) (width 0.2) (layer "F.Cu") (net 7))
 (segment (start 180.2167 97.818) (end 177.051 100.9837) (width 0.2) (layer "F.Cu") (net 7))
 (segment (start 178.0027 102.616) (end 178.2475 102.616) (width 0.2) (layer "F.Cu") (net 7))
 (segment (start 177.051 101.6643) (end 178.0027 102.616) (width 0.2) (layer "F.Cu") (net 7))
 (segment (start 183.079 103.914) (end 180.511 101.346) (width 0.2) (layer "F.Cu") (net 18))
 (segment (start 180.511 101.346) (end 178.2475 101.346) (width 0.2) (layer "F.Cu") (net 18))
 (segment (start 181.273 107.696) (end 183.079 109.502) (width 0.2) (layer "F.Cu") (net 14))
 (segment (start 183.587 115.09) (end 183.079 114.582) (width 0.2) (layer "F.Cu") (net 14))
 (segment (start 183.079 114.582) (end 183.079 109.502) (width 0.2) (layer "F.Cu") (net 14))
 (segment (start 178.2475 107.696) (end 181.273 107.696) (width 0.2) (layer "F.Cu") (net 14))
 (segment (start 171.9054 108.043) (end 172.8284 108.966) (width 0.2) (layer "F.Cu") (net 2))
 (segment (start 173.8682 108.966) (end 178.0815 113.1793) (width 0.2) (layer "F.Cu") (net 2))
 (segment (start 170.9355 104.1861) (end 171.9054 105.156) (width 0.2) (layer "F.Cu") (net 2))
 (segment (start 171.9054 105.156) (end 173.0975 105.156) (width 0.2) (layer "F.Cu") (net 2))
 (segment (start 171.9054 105.156) (end 171.9054 108.043) (width 0.2) (layer "F.Cu") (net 2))
 (segment (start 158.496 105.664) (end 159.9739 104.1861) (width 0.2) (layer "F.Cu") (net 2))
 (segment (start 172.8284 108.966) (end 173.0975 108.966) (width 0.2) (layer "F.Cu") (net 2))
 (segment (start 159.9739 104.1861) (end 170.9355 104.1861) (width 0.2) (layer "F.Cu") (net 2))
 (segment (start 178.0815 114.356) (end 178.0815 113.1793) (width 0.2) (layer "F.Cu") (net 2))
 (segment (start 173.0975 108.966) (end 173.8682 108.966) (width 0.2) (layer "F.Cu") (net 2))
 (segment (start 167.132 105.664) (end 167.132 110.236) (width 0.2) (layer "F.Cu") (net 11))
 (segment (start 164.8051 111.76) (end 166.3291 110.236) (width 0.2) (layer "F.Cu") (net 11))
 (segment (start 164.8051 111.7951) (end 164.8051 111.76) (width 0.2) (layer "F.Cu") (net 11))
 (segment (start 170.132 117.122) (end 164.8051 111.7951) (width 0.2) (layer "F.Cu") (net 11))
 (segment (start 166.3291 110.236) (end 167.132 110.236) (width 0.2) (layer "F.Cu") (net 11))
 (segment (start 164.8051 111.76) (end 162.807 111.76) (width 0.2) (layer "F.Cu") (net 11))
 (segment (start 167.132 110.236) (end 173.0975 110.236) (width 0.2) (layer "F.Cu") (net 11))
 (segment (start 173.4408 114.9293) (end 173.2712 115.0989) (width 0.2) (layer "F.Cu") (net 15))
 (segment (start 173.4408 114.9293) (end 175.0815 114.9293) (width 0.2) (layer "F.Cu") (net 15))
 (segment (start 175.0815 116.106) (end 175.0815 114.9293) (width 0.2) (layer "F.Cu") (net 15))
 (segment (start 167.2545 93.754) (end 167.2545 94.5392) (width 0.2) (layer "F.Cu") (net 15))
 (segment (start 173.2712 115.0989) (end 173.4408 114.9293) (width 0.2) (layer "F.Cu") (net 15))
 (segment (start 167.2545 94.5392) (end 167.4503 94.735) (width 0.2) (layer "F.Cu") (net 15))
 (segment (start 173.2712 115.0989) (end 173.4408 114.9293) (width 0.2) (layer "F.Cu") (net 15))
 (via (at 173.2712 115.0989) (size 0.6) (drill 0.3) (layers "F.Cu" "B.Cu") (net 15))
 (via (at 167.4503 94.735) (size 0.6) (drill 0.3) (layers "F.Cu" "B.Cu") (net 15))
 (segment (start 167.4503 101.2681) (end 167.4503 94.735) (width 0.2) (layer "B.Cu") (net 15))
 (segment (start 173.2712 115.0989) (end 173.4408 114.9293) (width 0.2) (layer "B.Cu") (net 15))
 (segment (start 173.4408 114.9293) (end 173.2712 115.0989) (width 0.2) (layer "B.Cu") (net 15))
 (segment (start 174.2072 108.025) (end 167.4503 101.2681) (width 0.2) (layer "B.Cu") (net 15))
 (segment (start 173.2712 115.0989) (end 174.2072 114.1629) (width 0.2) (layer "B.Cu") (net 15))
 (segment (start 174.2072 114.1629) (end 174.2072 108.025) (width 0.2) (layer "B.Cu") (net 15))
 (segment (start 178.635 116.106) (end 179.7283 115.0127) (width 0.2) (layer "F.Cu") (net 17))
 (segment (start 177.0815 116.106) (end 178.635 116.106) (width 0.2) (layer "F.Cu") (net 17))
 (segment (start 178.7701 103.3634) (end 178.2475 103.886) (width 0.2) (layer "F.Cu") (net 17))
 (segment (start 180.6371 103.3634) (end 178.7701 103.3634) (width 0.2) (layer "F.Cu") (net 17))
 (via (at 179.7283 115.0127) (size 0.6) (drill 0.3) (layers "F.Cu" "B.Cu") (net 17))
 (via (at 180.6371 103.3634) (size 0.6) (drill 0.3) (layers "F.Cu" "B.Cu") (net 17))
 (segment (start 180.7258 103.4521) (end 180.6371 103.3634) (width 0.2) (layer "B.Cu") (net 17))
 (segment (start 179.7283 115.0127) (end 180.7258 114.0152) (width 0.2) (layer "B.Cu") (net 17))
 (segment (start 180.7258 114.0152) (end 180.7258 103.4521) (width 0.2) (layer "B.Cu") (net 17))
 (segment (start 173.7625 113.1793) (end 172.7744 114.1674) (width 0.2) (layer "F.Cu") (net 5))
 (segment (start 172.7744 114.1674) (end 173.7625 113.1793) (width 0.2) (layer "F.Cu") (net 5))
 (segment (start 172.7732 114.1662) (end 172.7744 114.1674) (width 0.2) (layer "F.Cu") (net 5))
 (segment (start 163.1703 93.5268) (end 163.3975 93.754) (width 0.2) (layer "F.Cu") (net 5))
 (segment (start 176.0815 114.356) (end 176.0815 113.1793) (width 0.2) (layer "F.Cu") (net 5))
 (segment (start 172.7744 114.1674) (end 172.7732 114.1662) (width 0.2) (layer "F.Cu") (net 5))
 (segment (start 162.3298 93.5268) (end 163.1703 93.5268) (width 0.2) (layer "F.Cu") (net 5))
 (segment (start 173.7625 113.1793) (end 176.0815 113.1793) (width 0.2) (layer "F.Cu") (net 5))
 (segment (start 172.7744 114.1674) (end 173.7625 113.1793) (width 0.2) (layer "F.Cu") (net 5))
 (via (at 172.7744 114.1674) (size 0.6) (drill 0.3) (layers "F.Cu" "B.Cu") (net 5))
 (via (at 162.3298 93.5268) (size 0.6) (drill 0.3) (layers "F.Cu" "B.Cu") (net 5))
 (segment (start 172.7732 114.1662) (end 172.7744 114.1674) (width 0.2) (layer "B.Cu") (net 5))
 (segment (start 162.3298 93.5268) (end 162.3298 103.7228) (width 0.2) (layer "B.Cu") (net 5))
 (segment (start 172.7744 114.1674) (end 172.7732 114.1662) (width 0.2) (layer "B.Cu") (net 5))
 (segment (start 162.3298 103.7228) (end 172.7744 114.1674) (width 0.2) (layer "B.Cu") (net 5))
 (segment (start 158.1252 93.754) (end 149.1735 102.7057) (width 0.2) (layer "F.Cu") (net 3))
 (segment (start 159.437 93.754) (end 158.1252 93.754) (width 0.2) (layer "F.Cu") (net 3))
 (segment (start 149.1735 102.7057) (end 149.1735 103.222) (width 0.2) (layer "F.Cu") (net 3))
 (segment (start 173.0975 102.616) (end 173.3621 102.616) (width 0.2) (layer "F.Cu") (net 6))
 (segment (start 174.2842 100.9871) (end 173.7897 100.4926) (width 0.2) (layer "F.Cu") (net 6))
 (segment (start 171.9611 100.4926) (end 165.2225 93.754) (width 0.2) (layer "F.Cu") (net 6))
 (segment (start 173.7897 100.4926) (end 171.9611 100.4926) (width 0.2) (layer "F.Cu") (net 6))
 (segment (start 173.3621 102.616) (end 174.2842 101.6939) (width 0.2) (layer "F.Cu") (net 6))
 (segment (start 174.2842 101.6939) (end 174.2842 100.9871) (width 0.2) (layer "F.Cu") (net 6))
 (segment (start 176.202 101.555) (end 176.3668 101.7198) (width 0.2) (layer "F.Cu") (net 16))
 (segment (start 176.3668 103.5718) (end 177.951 105.156) (width 0.2) (layer "F.Cu") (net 16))
 (segment (start 176.3668 101.7198) (end 176.3668 103.5718) (width 0.2) (layer "F.Cu") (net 16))
 (segment (start 177.951 105.156) (end 178.2475 105.156) (width 0.2) (layer "F.Cu") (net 16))
 (segment (start 169.0795 93.754) (end 176.202 100.8765) (width 0.2) (layer "F.Cu") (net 16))
 (segment (start 176.202 101.555) (end 176.3668 101.7198) (width 0.2) (layer "F.Cu") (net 16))
 (segment (start 176.202 100.8765) (end 176.202 101.555) (width 0.2) (layer "F.Cu") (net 16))
 (segment (start 177.93 106.7435) (end 178.2475 106.426) (width 0.2) (layer "F.Cu") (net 10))
 (segment (start 171.0175 93.754) (end 171.0175 94.7539) (width 0.2) (layer "F.Cu") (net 10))
 (segment (start 174.7182 106.7435) (end 177.93 106.7435) (width 0.2) (layer "F.Cu") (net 10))
 (via (at 171.0175 94.7539) (size 0.6) (drill 0.3) (layers "F.Cu" "B.Cu") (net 10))
 (via (at 174.7182 106.7435) (size 0.6) (drill 0.3) (layers "F.Cu" "B.Cu") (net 10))
 (segment (start 174.7182 98.4546) (end 174.7182 106.7435) (width 0.2) (layer "B.Cu") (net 10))
 (segment (start 171.0175 94.7539) (end 174.7182 98.4546) (width 0.2) (layer "B.Cu") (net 10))
 (segment (start 154.0645 114.0155) (end 157.171 117.122) (width 0.2) (layer "F.Cu") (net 8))
 (segment (start 175.7956 108.3092) (end 175.1824 107.696) (width 0.2) (layer "F.Cu") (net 8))
 (segment (start 175.1824 107.696) (end 173.0975 107.696) (width 0.2) (layer "F.Cu") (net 8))
 (segment (start 154.0645 111.76) (end 154.0645 114.0155) (width 0.2) (layer "F.Cu") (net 8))
 (segment (start 158.6236 118.5746) (end 176.4978 118.5746) (width 0.2) (layer "F.Cu") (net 8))
 (segment (start 157.171 117.122) (end 158.6236 118.5746) (width 0.2) (layer "F.Cu") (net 8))
 (via (at 175.7956 108.3092) (size 0.6) (drill 0.3) (layers "F.Cu" "B.Cu") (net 8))
 (via (at 176.4978 118.5746) (size 0.6) (drill 0.3) (layers "F.Cu" "B.Cu") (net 8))
 (segment (start 175.6103 108.4945) (end 175.6103 117.6871) (width 0.2) (layer "B.Cu") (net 8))
 (segment (start 175.6103 117.6871) (end 176.4978 118.5746) (width 0.2) (layer "B.Cu") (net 8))
 (segment (start 175.7956 108.3092) (end 175.6103 108.4945) (width 0.2) (layer "B.Cu") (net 8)))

